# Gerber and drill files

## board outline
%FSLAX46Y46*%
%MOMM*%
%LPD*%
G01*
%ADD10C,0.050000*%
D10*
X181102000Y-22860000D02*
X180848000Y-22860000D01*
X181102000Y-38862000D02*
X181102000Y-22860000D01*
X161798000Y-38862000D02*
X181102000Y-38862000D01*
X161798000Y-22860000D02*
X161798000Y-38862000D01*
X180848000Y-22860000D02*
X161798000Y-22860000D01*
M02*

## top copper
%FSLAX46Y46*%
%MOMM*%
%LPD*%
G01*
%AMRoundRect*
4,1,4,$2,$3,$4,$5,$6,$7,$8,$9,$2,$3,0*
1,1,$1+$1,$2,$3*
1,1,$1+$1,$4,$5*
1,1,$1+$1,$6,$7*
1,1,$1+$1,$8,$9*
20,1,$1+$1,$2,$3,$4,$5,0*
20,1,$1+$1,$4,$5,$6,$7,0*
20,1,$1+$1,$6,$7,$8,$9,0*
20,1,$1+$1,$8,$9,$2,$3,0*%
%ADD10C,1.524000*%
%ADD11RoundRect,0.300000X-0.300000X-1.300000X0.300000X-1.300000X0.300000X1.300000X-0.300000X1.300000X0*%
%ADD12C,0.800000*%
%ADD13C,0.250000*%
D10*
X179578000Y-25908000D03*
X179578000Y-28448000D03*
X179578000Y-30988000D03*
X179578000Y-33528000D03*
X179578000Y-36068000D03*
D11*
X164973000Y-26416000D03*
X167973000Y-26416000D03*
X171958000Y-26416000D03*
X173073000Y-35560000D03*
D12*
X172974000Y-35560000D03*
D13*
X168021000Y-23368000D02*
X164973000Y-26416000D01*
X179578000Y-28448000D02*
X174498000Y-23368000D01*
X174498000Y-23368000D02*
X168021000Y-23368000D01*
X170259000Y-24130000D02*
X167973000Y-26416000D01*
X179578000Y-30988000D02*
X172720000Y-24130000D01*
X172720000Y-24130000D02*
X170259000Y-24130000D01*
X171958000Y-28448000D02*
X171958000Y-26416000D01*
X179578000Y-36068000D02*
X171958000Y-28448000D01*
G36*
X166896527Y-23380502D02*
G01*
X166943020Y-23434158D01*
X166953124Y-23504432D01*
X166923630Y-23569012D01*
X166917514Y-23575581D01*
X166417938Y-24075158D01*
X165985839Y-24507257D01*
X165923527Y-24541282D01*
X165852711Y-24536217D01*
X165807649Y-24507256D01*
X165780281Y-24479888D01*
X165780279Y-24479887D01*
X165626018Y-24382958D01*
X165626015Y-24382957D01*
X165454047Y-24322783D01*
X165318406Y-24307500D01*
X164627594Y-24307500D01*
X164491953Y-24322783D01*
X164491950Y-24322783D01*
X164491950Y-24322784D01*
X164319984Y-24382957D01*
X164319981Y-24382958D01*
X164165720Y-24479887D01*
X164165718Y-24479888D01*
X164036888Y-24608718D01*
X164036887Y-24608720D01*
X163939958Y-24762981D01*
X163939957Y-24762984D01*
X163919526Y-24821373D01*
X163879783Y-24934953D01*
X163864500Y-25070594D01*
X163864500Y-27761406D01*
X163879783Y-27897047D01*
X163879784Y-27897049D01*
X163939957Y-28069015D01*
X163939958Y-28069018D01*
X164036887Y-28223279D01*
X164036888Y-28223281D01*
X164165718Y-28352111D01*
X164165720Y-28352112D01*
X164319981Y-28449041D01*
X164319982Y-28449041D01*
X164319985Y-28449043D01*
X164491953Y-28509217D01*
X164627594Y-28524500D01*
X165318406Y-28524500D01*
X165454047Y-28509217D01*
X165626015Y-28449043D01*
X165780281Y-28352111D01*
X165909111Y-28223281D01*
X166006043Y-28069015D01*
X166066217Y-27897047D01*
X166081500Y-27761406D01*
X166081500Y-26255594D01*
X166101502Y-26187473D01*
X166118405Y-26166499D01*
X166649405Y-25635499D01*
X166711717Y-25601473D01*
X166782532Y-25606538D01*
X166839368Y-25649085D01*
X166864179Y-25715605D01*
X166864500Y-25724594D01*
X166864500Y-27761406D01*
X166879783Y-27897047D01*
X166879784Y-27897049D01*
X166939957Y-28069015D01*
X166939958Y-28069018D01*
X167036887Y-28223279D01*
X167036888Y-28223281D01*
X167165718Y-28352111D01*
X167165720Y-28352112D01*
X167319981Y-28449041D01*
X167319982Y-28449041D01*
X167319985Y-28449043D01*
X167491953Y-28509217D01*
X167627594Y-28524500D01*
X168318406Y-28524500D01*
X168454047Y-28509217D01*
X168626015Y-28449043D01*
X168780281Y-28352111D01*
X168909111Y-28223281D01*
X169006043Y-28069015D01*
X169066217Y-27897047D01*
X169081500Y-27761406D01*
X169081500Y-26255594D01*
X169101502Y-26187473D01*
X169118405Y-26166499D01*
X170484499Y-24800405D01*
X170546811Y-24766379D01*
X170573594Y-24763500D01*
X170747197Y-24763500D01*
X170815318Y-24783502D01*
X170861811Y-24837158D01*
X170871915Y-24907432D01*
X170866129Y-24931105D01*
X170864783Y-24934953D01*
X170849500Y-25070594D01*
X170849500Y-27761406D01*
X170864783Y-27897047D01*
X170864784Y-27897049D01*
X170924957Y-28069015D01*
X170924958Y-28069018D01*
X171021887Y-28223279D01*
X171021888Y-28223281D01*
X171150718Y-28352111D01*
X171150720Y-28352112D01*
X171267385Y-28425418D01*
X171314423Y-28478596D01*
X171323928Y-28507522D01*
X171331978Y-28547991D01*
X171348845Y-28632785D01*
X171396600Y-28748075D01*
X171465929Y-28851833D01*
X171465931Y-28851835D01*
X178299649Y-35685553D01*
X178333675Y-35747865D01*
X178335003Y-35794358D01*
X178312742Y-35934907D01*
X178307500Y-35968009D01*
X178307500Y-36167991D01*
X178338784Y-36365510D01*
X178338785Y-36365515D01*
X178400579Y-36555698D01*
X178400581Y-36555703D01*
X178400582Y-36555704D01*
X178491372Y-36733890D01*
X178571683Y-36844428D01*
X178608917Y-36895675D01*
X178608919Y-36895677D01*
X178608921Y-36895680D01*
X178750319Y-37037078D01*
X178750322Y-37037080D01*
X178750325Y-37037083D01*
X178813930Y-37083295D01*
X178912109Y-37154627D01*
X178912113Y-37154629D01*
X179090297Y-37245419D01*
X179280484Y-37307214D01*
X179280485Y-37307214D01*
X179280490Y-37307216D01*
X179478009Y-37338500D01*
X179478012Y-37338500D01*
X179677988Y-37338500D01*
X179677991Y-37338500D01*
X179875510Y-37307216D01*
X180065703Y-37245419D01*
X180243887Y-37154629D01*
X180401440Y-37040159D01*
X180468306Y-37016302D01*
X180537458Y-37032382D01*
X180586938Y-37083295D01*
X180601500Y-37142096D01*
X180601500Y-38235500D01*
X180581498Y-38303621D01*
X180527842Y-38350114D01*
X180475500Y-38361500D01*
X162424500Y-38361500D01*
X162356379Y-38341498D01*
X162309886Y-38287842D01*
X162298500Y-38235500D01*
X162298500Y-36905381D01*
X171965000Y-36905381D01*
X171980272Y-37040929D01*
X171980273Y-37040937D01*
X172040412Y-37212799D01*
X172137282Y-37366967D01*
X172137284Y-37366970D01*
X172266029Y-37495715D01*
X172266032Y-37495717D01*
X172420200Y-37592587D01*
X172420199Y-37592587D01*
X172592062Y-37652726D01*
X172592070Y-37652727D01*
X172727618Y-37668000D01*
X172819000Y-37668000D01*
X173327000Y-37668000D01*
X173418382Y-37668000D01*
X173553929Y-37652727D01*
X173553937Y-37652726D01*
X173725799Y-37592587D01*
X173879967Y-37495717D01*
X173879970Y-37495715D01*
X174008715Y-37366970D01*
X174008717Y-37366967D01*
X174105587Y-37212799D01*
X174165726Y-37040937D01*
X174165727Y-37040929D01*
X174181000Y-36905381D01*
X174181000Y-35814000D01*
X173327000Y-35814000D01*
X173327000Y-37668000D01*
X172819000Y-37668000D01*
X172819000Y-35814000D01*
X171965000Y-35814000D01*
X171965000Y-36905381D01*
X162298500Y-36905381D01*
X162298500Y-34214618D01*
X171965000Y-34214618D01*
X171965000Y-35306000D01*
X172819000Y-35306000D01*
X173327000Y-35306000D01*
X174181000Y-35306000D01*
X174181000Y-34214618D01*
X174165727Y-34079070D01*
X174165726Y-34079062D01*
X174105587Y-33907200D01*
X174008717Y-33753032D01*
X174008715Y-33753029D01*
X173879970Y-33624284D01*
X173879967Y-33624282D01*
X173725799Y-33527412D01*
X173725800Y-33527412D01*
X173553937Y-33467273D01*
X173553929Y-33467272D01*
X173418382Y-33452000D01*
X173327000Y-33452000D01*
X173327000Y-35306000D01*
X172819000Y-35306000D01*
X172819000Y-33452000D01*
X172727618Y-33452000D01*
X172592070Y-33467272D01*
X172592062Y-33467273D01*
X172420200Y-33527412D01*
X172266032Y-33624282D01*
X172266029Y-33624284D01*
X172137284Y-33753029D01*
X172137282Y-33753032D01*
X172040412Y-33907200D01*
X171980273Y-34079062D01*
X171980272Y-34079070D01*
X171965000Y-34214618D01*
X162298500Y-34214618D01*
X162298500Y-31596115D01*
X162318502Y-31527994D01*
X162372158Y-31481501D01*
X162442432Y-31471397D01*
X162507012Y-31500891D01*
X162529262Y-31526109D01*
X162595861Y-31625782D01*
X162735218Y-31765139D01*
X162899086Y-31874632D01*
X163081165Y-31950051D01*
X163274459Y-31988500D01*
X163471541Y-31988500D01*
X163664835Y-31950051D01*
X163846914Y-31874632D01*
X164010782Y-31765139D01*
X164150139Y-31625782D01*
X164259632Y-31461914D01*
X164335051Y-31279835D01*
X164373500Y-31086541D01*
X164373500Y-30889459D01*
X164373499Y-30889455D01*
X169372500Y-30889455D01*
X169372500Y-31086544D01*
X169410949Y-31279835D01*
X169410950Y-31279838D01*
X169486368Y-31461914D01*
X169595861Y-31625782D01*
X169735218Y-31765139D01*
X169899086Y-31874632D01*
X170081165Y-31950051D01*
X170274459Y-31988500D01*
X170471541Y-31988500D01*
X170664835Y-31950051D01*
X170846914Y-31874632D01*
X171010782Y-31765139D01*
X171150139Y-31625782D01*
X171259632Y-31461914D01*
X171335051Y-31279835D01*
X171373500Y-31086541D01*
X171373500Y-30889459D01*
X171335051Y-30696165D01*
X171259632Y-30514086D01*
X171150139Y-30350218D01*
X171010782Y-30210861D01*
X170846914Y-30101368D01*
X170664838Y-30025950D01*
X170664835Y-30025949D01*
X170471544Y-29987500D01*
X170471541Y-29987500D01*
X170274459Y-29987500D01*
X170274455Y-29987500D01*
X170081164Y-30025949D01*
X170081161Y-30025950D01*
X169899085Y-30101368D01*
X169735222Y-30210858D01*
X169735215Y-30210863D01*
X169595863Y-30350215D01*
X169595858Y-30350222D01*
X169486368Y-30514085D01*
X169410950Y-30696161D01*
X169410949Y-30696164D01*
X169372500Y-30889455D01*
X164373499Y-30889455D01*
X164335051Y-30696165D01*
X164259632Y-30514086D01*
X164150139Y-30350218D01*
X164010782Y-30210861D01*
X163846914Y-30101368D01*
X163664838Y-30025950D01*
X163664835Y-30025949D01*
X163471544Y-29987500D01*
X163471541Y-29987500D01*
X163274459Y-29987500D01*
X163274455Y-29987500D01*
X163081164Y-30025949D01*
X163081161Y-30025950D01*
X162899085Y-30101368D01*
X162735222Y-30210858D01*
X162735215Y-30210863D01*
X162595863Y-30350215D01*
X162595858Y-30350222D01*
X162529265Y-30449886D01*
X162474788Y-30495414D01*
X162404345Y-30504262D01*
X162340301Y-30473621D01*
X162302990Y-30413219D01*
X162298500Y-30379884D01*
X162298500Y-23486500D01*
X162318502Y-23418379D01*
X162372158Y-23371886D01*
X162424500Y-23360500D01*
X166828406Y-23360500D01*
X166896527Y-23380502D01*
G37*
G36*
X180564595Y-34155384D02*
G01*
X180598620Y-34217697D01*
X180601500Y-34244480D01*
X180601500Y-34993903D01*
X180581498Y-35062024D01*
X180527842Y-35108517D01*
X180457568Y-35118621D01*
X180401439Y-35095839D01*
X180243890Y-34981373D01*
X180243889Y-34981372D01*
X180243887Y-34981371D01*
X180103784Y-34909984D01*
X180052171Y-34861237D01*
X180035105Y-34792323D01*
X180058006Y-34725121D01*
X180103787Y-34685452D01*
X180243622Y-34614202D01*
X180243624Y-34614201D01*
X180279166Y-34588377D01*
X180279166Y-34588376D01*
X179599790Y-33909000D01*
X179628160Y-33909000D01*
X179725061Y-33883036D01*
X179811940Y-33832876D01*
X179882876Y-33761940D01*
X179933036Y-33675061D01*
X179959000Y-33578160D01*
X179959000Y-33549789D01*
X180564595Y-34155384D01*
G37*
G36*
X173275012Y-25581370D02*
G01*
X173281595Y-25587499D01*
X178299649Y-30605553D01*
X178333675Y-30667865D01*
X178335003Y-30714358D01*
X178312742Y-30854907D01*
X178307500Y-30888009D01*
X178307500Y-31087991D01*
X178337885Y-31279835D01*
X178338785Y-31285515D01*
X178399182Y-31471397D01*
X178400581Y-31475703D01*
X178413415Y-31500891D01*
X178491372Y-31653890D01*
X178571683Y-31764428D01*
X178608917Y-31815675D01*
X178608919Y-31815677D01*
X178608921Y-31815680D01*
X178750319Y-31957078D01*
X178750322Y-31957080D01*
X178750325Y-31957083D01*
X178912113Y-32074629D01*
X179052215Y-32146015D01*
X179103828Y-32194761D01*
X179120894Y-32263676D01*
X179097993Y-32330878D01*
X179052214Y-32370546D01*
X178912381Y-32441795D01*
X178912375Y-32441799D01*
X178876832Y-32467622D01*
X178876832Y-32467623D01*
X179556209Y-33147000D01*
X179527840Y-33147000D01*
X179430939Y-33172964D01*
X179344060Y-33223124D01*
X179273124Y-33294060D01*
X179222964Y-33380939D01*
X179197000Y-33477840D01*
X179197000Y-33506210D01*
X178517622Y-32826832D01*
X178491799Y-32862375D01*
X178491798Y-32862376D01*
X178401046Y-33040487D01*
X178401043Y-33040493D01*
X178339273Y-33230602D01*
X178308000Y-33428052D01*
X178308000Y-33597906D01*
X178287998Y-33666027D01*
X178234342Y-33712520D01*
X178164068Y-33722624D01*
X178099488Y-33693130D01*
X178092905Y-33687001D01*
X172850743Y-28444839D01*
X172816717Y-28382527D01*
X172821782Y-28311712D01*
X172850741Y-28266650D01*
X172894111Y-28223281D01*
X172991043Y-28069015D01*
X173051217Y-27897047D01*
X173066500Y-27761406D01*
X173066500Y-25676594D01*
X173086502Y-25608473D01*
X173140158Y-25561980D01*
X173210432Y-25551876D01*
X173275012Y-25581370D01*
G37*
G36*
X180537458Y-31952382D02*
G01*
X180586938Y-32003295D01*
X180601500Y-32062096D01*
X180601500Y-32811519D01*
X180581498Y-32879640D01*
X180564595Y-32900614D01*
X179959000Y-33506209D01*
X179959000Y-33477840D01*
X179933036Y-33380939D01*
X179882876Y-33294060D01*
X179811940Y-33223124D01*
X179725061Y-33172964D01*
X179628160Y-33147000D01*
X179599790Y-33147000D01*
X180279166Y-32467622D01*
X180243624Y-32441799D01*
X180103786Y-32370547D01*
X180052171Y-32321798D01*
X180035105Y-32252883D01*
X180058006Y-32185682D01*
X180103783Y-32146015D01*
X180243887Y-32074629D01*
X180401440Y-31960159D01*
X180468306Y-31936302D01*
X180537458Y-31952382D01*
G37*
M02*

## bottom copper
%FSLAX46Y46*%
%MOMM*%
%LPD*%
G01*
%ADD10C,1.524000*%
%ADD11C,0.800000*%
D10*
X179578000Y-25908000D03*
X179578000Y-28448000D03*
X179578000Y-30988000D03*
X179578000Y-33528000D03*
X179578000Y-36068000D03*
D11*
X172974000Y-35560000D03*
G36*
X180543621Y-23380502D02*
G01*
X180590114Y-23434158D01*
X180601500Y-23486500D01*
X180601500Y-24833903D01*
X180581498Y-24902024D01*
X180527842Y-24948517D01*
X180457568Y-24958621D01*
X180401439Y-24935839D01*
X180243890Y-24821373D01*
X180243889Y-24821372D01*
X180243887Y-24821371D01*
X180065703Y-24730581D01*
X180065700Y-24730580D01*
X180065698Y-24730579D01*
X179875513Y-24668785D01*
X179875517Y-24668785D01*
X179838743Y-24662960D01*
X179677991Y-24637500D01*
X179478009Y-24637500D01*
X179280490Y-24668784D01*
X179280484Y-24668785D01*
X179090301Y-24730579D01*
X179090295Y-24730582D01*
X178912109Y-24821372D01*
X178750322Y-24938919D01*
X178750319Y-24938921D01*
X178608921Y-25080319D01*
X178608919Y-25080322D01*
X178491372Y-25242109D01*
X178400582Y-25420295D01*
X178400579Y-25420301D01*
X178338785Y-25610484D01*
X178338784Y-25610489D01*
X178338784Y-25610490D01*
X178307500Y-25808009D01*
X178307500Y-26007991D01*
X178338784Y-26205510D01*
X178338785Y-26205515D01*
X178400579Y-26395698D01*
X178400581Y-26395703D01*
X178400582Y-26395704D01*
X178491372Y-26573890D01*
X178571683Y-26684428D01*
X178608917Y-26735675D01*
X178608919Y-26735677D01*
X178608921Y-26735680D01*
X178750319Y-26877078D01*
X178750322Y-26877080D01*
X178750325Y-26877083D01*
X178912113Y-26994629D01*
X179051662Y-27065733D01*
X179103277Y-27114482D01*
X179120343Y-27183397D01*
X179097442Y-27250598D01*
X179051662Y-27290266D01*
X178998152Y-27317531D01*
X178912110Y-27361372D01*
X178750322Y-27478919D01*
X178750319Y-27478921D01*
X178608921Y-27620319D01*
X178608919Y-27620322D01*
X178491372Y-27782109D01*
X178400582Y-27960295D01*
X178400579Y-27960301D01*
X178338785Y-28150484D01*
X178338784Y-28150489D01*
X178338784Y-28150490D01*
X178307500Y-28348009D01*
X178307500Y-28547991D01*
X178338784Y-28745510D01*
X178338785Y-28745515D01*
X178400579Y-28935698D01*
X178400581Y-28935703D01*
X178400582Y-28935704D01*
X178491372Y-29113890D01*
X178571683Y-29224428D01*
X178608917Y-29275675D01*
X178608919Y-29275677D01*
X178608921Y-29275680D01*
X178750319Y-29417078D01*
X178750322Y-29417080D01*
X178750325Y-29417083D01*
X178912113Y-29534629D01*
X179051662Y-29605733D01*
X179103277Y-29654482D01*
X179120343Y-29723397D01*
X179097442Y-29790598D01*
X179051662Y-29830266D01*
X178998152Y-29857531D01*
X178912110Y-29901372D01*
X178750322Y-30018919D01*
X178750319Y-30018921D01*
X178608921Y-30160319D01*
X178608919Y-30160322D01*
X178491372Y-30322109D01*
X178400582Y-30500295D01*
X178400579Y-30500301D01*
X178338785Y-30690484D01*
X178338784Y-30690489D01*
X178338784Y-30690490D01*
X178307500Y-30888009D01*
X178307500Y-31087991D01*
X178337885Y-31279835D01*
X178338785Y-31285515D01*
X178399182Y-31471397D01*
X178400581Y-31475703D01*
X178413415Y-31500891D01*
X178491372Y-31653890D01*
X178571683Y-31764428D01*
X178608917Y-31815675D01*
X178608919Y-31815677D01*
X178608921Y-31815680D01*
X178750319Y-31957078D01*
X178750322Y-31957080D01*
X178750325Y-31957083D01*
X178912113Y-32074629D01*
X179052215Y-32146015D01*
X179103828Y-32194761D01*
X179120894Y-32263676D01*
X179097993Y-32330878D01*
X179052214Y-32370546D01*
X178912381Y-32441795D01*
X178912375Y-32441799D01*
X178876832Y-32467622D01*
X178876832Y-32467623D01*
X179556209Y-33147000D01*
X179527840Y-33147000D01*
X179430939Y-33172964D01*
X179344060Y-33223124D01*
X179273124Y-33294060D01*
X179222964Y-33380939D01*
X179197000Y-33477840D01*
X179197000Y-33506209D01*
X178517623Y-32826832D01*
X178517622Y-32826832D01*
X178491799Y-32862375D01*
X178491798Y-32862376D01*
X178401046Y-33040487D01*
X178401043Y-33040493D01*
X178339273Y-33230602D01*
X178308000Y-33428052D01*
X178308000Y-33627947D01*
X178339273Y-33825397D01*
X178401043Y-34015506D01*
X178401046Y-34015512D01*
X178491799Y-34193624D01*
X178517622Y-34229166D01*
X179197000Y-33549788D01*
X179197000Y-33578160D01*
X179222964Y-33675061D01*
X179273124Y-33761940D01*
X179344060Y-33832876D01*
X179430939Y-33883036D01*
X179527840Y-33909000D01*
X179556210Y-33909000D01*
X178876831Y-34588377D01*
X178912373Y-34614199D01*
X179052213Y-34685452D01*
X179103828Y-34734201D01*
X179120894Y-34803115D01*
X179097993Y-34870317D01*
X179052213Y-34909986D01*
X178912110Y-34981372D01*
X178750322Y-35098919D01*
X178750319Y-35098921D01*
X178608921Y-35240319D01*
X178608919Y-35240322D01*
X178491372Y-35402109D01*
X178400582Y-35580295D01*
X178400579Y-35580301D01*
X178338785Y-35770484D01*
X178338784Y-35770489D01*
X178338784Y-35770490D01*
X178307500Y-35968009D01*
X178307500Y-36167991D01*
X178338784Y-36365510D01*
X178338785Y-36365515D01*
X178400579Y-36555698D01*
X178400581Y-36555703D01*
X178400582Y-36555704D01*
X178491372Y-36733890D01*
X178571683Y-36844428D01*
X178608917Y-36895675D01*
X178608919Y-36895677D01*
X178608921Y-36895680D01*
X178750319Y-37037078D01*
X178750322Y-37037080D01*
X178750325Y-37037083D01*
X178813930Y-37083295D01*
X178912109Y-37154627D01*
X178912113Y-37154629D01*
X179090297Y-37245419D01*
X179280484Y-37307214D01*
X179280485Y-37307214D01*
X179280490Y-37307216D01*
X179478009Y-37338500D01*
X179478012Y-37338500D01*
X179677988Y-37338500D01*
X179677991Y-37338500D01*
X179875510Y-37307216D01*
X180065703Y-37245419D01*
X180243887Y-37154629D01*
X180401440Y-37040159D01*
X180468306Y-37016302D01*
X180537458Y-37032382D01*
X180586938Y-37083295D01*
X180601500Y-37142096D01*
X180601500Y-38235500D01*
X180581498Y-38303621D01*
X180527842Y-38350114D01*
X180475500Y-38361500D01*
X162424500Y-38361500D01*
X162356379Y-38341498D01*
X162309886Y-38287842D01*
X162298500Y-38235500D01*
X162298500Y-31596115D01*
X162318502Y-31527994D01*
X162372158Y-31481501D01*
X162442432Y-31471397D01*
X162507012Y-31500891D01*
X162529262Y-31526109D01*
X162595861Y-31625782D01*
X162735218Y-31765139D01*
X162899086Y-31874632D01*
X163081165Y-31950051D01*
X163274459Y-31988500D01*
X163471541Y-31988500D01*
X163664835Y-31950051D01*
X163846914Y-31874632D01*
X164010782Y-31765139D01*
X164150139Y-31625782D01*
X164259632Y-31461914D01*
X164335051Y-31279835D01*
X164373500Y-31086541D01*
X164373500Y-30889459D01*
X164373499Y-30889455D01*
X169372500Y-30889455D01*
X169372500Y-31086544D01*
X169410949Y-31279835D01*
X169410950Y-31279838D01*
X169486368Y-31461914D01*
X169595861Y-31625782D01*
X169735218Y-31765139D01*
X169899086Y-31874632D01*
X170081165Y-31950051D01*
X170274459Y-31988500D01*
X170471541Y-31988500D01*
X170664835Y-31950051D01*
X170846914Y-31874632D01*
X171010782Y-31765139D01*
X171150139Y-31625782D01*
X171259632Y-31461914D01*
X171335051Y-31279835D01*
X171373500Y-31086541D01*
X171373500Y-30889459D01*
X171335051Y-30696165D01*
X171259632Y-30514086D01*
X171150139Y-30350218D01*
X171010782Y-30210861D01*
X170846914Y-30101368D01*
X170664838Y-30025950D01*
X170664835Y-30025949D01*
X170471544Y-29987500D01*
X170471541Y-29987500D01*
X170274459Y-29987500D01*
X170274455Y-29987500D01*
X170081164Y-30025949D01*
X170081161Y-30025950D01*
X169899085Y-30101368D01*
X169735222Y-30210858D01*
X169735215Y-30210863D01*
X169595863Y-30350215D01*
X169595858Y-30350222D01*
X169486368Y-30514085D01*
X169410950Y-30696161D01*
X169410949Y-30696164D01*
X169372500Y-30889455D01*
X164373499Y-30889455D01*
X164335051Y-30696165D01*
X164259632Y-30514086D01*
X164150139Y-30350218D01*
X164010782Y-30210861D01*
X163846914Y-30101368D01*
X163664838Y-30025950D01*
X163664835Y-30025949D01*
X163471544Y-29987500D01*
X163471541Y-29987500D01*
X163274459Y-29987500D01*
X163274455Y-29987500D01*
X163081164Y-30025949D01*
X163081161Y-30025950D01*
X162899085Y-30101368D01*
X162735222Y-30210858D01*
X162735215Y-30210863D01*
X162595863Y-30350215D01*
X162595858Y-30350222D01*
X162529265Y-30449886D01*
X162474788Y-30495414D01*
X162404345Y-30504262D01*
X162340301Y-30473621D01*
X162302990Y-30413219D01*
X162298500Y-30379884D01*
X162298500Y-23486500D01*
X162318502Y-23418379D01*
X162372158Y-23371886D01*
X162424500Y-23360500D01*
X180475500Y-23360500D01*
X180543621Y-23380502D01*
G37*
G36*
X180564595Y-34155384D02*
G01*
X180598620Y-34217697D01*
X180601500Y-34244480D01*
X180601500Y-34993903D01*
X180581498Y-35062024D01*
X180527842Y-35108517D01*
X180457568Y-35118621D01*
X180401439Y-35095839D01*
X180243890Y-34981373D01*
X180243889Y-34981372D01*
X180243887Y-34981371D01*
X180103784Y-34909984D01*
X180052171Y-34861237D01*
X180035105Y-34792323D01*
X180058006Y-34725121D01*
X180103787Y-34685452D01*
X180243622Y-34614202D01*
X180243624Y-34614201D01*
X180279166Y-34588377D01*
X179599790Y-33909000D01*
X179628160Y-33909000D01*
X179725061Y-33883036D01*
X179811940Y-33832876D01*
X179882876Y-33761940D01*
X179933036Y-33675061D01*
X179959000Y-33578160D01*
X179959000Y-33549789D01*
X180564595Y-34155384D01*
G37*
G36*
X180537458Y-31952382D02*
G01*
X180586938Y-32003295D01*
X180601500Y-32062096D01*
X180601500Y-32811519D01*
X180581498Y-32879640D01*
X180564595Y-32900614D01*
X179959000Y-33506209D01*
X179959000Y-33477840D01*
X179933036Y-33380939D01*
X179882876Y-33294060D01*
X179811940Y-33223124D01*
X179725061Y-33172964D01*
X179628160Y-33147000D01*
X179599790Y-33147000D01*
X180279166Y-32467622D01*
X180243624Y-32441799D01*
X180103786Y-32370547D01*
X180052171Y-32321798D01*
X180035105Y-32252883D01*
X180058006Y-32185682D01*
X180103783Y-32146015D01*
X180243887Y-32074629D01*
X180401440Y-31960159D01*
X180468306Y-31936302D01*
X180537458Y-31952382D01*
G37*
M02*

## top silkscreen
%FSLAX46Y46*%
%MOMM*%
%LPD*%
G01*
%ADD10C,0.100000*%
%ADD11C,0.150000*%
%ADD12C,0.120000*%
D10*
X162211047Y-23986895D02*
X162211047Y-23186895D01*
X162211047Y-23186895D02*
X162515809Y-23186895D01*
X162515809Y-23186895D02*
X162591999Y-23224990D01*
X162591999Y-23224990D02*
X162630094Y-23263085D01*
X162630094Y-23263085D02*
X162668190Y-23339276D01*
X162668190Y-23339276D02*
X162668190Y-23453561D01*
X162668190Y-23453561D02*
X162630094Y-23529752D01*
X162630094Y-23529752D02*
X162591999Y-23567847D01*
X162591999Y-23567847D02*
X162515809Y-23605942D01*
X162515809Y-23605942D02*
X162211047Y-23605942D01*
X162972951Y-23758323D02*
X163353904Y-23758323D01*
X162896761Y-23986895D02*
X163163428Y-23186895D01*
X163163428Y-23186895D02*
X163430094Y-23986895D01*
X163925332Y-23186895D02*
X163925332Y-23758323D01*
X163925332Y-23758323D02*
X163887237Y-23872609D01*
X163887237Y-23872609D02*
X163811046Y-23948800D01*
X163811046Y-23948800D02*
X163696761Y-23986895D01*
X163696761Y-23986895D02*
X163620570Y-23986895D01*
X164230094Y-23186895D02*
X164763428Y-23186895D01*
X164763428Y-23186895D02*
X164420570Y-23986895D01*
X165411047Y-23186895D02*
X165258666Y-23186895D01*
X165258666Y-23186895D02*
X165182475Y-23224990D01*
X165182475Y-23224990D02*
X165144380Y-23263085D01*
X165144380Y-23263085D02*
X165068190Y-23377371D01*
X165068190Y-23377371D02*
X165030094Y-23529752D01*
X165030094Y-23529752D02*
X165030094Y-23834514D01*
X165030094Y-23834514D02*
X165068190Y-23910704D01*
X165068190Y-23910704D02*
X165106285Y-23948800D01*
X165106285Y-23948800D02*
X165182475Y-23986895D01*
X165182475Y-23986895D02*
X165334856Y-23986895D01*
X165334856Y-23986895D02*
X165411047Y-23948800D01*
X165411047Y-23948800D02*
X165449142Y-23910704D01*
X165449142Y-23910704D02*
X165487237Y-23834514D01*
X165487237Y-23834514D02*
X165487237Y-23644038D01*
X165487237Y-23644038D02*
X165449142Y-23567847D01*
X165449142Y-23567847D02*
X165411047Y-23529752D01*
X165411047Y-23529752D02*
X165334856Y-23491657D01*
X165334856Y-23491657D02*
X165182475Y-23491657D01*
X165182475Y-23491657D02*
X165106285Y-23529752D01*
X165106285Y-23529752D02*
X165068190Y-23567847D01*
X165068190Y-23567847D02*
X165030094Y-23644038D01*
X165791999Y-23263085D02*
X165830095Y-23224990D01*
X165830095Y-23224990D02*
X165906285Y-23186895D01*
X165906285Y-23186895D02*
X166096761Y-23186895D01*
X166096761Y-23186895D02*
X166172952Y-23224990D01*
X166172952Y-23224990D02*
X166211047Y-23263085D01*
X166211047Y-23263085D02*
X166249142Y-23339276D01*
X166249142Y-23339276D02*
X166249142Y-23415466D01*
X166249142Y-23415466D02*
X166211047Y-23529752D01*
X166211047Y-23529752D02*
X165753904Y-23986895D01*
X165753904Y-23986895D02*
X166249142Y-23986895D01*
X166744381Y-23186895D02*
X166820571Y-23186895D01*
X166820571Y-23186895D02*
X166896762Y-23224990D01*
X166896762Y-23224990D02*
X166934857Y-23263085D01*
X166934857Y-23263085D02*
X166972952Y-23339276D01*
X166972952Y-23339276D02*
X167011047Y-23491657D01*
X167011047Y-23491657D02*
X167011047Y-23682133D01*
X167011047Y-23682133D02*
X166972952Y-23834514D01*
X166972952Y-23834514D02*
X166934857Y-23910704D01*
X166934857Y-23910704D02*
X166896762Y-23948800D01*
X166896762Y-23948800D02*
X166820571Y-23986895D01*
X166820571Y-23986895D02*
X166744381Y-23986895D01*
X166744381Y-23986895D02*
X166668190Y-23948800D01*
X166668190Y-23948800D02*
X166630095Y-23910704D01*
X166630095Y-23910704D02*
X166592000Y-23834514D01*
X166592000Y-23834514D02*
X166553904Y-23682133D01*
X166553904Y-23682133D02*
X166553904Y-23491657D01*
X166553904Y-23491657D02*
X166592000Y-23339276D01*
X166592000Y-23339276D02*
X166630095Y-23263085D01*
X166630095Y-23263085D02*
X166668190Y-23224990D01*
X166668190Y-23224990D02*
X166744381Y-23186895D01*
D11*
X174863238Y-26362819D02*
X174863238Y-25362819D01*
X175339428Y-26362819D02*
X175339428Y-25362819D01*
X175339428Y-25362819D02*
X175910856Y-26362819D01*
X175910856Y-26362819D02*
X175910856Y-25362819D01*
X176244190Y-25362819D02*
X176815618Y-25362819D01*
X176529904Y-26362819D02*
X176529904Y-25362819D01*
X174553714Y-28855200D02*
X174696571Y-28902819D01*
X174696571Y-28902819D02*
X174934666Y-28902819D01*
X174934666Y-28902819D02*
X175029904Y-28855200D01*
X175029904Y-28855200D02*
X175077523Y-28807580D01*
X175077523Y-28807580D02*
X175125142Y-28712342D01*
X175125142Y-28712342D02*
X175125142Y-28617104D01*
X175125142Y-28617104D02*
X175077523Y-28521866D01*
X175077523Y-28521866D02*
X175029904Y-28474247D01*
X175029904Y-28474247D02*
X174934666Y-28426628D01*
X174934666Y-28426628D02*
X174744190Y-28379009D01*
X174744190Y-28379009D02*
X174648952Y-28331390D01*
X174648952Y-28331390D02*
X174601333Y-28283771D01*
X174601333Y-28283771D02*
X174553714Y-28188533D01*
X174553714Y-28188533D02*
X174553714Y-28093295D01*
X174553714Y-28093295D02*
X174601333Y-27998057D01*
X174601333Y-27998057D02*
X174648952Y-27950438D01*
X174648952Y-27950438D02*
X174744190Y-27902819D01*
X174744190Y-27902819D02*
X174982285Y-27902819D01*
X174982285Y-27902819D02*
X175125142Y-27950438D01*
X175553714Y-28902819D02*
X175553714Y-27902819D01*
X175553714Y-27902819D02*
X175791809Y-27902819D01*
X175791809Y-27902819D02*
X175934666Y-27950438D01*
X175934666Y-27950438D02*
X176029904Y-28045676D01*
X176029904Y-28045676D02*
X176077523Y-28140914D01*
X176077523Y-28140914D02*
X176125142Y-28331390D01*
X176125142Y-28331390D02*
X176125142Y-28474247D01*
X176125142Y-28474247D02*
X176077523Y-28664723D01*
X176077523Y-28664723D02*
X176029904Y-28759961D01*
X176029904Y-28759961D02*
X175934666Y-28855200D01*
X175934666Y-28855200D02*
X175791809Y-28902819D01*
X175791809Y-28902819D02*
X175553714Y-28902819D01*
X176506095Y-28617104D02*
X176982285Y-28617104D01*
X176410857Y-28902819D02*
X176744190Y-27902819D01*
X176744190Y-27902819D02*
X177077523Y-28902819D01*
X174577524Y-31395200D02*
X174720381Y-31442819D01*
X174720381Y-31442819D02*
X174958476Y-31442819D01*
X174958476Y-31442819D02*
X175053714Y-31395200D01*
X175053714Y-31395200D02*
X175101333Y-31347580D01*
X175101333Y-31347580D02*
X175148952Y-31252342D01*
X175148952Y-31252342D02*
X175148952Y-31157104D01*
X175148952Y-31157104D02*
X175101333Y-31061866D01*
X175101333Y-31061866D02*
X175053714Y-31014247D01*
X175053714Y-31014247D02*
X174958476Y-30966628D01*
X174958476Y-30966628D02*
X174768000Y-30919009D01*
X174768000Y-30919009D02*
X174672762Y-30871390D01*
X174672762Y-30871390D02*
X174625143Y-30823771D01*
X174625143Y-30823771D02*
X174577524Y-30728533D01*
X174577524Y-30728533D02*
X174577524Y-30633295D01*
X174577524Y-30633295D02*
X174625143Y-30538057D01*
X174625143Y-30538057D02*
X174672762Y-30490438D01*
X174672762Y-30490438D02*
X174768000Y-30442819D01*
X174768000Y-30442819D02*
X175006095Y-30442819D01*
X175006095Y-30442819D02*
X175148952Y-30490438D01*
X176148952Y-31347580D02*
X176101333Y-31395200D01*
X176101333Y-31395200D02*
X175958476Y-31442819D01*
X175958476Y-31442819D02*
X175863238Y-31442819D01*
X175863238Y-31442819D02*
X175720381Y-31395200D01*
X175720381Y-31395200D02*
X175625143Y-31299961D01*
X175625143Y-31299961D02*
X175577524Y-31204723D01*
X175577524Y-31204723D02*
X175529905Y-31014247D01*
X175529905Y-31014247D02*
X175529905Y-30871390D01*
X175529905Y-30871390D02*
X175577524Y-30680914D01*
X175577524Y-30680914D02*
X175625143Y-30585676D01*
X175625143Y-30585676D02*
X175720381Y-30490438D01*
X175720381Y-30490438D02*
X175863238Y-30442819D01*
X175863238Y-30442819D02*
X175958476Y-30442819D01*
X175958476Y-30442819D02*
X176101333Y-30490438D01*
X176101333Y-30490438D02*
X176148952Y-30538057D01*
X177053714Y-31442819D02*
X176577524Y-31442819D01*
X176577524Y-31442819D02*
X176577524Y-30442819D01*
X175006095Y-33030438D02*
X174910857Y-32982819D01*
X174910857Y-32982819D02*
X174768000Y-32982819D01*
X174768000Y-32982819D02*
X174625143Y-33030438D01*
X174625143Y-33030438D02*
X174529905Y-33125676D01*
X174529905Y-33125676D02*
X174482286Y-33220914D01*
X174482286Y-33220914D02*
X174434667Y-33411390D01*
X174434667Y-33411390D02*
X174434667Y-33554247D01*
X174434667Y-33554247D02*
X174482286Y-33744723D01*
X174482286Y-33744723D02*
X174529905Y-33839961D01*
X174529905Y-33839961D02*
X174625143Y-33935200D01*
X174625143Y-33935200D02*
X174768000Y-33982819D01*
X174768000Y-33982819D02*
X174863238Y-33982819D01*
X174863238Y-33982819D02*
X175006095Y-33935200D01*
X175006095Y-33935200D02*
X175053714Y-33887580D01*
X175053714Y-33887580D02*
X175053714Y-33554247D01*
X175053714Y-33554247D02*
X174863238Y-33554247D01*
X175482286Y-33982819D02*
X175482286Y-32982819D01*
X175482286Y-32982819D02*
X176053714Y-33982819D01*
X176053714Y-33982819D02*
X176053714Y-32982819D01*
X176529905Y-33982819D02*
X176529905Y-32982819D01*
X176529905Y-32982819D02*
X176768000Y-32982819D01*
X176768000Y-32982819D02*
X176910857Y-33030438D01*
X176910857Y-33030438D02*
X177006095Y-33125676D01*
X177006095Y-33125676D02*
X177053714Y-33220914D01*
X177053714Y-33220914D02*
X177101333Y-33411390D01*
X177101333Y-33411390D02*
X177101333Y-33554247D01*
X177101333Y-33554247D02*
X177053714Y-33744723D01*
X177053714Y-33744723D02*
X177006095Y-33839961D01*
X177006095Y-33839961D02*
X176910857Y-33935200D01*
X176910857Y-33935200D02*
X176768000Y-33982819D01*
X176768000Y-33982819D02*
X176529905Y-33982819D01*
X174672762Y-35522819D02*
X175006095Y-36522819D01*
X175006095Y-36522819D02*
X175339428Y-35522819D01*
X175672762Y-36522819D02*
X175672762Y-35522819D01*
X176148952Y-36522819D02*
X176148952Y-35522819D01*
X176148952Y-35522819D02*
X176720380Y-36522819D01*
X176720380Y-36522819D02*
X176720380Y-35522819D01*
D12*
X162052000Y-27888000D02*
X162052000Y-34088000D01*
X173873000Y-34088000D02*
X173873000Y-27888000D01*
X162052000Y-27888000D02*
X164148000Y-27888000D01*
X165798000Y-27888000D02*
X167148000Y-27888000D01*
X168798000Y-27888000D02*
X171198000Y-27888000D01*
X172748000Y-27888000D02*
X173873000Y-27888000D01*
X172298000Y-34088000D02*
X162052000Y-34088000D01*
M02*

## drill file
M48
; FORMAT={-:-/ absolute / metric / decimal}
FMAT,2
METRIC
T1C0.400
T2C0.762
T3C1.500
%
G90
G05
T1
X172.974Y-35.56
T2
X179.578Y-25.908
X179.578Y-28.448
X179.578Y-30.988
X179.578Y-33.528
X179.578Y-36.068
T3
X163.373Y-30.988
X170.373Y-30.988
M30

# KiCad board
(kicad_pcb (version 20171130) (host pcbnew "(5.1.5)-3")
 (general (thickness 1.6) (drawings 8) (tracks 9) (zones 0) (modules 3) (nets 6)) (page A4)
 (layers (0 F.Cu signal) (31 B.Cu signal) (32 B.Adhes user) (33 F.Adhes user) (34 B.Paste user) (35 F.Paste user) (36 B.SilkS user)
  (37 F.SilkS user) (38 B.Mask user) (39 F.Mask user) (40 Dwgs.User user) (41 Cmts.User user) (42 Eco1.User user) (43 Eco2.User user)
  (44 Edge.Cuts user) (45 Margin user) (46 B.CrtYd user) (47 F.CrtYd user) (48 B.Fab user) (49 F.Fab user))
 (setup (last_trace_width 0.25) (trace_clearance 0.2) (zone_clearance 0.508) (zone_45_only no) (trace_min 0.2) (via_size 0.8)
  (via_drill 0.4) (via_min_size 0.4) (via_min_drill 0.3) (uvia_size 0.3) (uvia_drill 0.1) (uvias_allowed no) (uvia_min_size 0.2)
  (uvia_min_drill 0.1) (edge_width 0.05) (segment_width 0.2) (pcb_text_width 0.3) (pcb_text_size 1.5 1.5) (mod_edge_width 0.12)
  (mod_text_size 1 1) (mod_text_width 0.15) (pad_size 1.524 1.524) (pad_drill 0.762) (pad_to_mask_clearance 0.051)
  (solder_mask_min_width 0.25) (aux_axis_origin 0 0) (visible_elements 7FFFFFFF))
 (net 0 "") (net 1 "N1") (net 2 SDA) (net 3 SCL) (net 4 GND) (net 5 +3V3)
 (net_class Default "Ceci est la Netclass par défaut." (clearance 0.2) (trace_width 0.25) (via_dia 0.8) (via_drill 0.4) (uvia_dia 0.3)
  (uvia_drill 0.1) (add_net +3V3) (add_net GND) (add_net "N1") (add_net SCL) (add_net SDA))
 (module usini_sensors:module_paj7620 (layer F.Cu) (at 179.578 23.368 180)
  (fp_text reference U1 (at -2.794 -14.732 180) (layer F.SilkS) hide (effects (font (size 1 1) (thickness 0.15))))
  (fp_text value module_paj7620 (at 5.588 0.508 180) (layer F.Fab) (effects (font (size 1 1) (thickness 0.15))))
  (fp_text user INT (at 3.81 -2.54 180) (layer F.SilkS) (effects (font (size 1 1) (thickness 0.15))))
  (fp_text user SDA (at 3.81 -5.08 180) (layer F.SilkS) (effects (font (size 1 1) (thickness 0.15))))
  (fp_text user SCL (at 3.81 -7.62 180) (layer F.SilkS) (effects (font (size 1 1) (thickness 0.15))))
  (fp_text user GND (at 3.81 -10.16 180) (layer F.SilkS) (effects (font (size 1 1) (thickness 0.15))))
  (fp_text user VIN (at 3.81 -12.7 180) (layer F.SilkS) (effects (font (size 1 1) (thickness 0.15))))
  (pad 5 thru_hole circle (at 0 -2.54 180) (size 1.524 1.524) (drill 0.762) (layers *.Cu *.Mask) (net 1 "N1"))
  (pad 4 thru_hole circle (at 0 -5.08 180) (size 1.524 1.524) (drill 0.762) (layers *.Cu *.Mask) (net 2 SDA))
  (pad 3 thru_hole circle (at 0 -7.62 180) (size 1.524 1.524) (drill 0.762) (layers *.Cu *.Mask) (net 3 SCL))
  (pad 2 thru_hole circle (at 0 -10.16 180) (size 1.524 1.524) (drill 0.762) (layers *.Cu *.Mask) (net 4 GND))
  (pad 1 thru_hole circle (at 0 -12.7 180) (size 1.524 1.524) (drill 0.762) (layers *.Cu *.Mask) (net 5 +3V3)))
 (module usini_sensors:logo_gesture (layer B.Cu) (at 171.45 26.416 180)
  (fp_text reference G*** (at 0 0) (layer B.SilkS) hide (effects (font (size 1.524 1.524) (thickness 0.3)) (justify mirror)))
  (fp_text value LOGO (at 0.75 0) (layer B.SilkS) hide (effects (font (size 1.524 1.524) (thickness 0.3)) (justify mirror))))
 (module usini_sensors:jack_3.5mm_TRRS (layer F.Cu) (at 168.148 30.988)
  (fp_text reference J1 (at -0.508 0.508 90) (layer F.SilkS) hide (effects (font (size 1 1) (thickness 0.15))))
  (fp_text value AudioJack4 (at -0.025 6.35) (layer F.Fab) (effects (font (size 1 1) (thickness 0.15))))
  (fp_line (start -6.096 -3.1) (end -6.096 3.1) (layer F.SilkS) (width 0.12))
  (fp_line (start 5.725 3.1) (end 5.725 -3.1) (layer F.SilkS) (width 0.12))
  (fp_line (start -6.096 -3.1) (end -4 -3.1) (layer F.SilkS) (width 0.12))
  (fp_line (start -2.35 -3.1) (end -1 -3.1) (layer F.SilkS) (width 0.12))
  (fp_line (start 0.65 -3.1) (end 3.05 -3.1) (layer F.SilkS) (width 0.12))
  (fp_line (start 4.6 -3.1) (end 5.725 -3.1) (layer F.SilkS) (width 0.12))
  (fp_line (start 4.15 3.1) (end -6.096 3.1) (layer F.SilkS) (width 0.12))
  (pad "" np_thru_hole circle (at 2.225 0) (size 1.5 1.5) (drill 1.5) (layers *.Cu *.Mask))
  (pad "" np_thru_hole circle (at -4.775 0) (size 1.5 1.5) (drill 1.5) (layers *.Cu *.Mask))
  (pad R2 smd roundrect (at -3.175 -4.572) (size 1.2 3.2) (layers F.Cu F.Paste F.Mask) (roundrect_rratio 0.25) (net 2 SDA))
  (pad R1 smd roundrect (at -0.175 -4.572) (size 1.2 3.2) (layers F.Cu F.Paste F.Mask) (roundrect_rratio 0.25) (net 3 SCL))
  (pad T smd roundrect (at 3.81 -4.572) (size 1.2 3.2) (layers F.Cu F.Paste F.Mask) (roundrect_rratio 0.25) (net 5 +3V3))
  (pad S smd roundrect (at 4.925 4.572) (size 1.2 3.2) (layers F.Cu F.Paste F.Mask) (roundrect_rratio 0.25) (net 4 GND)))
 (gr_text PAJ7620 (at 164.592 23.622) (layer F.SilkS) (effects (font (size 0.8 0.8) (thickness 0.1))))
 (gr_line (start 181.102 22.86) (end 180.848 22.86) (layer Edge.Cuts) (width 0.05))
 (gr_line (start 181.102 38.862) (end 181.102 22.86) (layer Edge.Cuts) (width 0.05))
 (gr_line (start 161.798 38.862) (end 181.102 38.862) (layer Edge.Cuts) (width 0.05))
 (gr_line (start 161.798 22.86) (end 161.798 38.862) (layer Edge.Cuts) (width 0.05))
 (gr_line (start 180.848 22.86) (end 161.798 22.86) (layer Edge.Cuts) (width 0.05))
 (via (at 172.974 35.56) (size 0.8) (drill 0.4) (layers F.Cu B.Cu) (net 4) (status 30))
 (segment (start 168.021 23.368) (end 164.973 26.416) (width 0.25) (layer F.Cu) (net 2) (status 20))
 (segment (start 179.578 28.448) (end 174.498 23.368) (width 0.25) (layer F.Cu) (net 2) (status 10))
 (segment (start 174.498 23.368) (end 168.021 23.368) (width 0.25) (layer F.Cu) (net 2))
 (segment (start 170.259 24.13) (end 167.973 26.416) (width 0.25) (layer F.Cu) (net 3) (status 20))
 (segment (start 179.578 30.988) (end 172.72 24.13) (width 0.25) (layer F.Cu) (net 3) (status 10))
 (segment (start 172.72 24.13) (end 170.259 24.13) (width 0.25) (layer F.Cu) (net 3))
 (segment (start 171.958 28.448) (end 171.958 26.416) (width 0.25) (layer F.Cu) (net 5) (status 20))
 (segment (start 179.578 36.068) (end 171.958 28.448) (width 0.25) (layer F.Cu) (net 5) (status 10))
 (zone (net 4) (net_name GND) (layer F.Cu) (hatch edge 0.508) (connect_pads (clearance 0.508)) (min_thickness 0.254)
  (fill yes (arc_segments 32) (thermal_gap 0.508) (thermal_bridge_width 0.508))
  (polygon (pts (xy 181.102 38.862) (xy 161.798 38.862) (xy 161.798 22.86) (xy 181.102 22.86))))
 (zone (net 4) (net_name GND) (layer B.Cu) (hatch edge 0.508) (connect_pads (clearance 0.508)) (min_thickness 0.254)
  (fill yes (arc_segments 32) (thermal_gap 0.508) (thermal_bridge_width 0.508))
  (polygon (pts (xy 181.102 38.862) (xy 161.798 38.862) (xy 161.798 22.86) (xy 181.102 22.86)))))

